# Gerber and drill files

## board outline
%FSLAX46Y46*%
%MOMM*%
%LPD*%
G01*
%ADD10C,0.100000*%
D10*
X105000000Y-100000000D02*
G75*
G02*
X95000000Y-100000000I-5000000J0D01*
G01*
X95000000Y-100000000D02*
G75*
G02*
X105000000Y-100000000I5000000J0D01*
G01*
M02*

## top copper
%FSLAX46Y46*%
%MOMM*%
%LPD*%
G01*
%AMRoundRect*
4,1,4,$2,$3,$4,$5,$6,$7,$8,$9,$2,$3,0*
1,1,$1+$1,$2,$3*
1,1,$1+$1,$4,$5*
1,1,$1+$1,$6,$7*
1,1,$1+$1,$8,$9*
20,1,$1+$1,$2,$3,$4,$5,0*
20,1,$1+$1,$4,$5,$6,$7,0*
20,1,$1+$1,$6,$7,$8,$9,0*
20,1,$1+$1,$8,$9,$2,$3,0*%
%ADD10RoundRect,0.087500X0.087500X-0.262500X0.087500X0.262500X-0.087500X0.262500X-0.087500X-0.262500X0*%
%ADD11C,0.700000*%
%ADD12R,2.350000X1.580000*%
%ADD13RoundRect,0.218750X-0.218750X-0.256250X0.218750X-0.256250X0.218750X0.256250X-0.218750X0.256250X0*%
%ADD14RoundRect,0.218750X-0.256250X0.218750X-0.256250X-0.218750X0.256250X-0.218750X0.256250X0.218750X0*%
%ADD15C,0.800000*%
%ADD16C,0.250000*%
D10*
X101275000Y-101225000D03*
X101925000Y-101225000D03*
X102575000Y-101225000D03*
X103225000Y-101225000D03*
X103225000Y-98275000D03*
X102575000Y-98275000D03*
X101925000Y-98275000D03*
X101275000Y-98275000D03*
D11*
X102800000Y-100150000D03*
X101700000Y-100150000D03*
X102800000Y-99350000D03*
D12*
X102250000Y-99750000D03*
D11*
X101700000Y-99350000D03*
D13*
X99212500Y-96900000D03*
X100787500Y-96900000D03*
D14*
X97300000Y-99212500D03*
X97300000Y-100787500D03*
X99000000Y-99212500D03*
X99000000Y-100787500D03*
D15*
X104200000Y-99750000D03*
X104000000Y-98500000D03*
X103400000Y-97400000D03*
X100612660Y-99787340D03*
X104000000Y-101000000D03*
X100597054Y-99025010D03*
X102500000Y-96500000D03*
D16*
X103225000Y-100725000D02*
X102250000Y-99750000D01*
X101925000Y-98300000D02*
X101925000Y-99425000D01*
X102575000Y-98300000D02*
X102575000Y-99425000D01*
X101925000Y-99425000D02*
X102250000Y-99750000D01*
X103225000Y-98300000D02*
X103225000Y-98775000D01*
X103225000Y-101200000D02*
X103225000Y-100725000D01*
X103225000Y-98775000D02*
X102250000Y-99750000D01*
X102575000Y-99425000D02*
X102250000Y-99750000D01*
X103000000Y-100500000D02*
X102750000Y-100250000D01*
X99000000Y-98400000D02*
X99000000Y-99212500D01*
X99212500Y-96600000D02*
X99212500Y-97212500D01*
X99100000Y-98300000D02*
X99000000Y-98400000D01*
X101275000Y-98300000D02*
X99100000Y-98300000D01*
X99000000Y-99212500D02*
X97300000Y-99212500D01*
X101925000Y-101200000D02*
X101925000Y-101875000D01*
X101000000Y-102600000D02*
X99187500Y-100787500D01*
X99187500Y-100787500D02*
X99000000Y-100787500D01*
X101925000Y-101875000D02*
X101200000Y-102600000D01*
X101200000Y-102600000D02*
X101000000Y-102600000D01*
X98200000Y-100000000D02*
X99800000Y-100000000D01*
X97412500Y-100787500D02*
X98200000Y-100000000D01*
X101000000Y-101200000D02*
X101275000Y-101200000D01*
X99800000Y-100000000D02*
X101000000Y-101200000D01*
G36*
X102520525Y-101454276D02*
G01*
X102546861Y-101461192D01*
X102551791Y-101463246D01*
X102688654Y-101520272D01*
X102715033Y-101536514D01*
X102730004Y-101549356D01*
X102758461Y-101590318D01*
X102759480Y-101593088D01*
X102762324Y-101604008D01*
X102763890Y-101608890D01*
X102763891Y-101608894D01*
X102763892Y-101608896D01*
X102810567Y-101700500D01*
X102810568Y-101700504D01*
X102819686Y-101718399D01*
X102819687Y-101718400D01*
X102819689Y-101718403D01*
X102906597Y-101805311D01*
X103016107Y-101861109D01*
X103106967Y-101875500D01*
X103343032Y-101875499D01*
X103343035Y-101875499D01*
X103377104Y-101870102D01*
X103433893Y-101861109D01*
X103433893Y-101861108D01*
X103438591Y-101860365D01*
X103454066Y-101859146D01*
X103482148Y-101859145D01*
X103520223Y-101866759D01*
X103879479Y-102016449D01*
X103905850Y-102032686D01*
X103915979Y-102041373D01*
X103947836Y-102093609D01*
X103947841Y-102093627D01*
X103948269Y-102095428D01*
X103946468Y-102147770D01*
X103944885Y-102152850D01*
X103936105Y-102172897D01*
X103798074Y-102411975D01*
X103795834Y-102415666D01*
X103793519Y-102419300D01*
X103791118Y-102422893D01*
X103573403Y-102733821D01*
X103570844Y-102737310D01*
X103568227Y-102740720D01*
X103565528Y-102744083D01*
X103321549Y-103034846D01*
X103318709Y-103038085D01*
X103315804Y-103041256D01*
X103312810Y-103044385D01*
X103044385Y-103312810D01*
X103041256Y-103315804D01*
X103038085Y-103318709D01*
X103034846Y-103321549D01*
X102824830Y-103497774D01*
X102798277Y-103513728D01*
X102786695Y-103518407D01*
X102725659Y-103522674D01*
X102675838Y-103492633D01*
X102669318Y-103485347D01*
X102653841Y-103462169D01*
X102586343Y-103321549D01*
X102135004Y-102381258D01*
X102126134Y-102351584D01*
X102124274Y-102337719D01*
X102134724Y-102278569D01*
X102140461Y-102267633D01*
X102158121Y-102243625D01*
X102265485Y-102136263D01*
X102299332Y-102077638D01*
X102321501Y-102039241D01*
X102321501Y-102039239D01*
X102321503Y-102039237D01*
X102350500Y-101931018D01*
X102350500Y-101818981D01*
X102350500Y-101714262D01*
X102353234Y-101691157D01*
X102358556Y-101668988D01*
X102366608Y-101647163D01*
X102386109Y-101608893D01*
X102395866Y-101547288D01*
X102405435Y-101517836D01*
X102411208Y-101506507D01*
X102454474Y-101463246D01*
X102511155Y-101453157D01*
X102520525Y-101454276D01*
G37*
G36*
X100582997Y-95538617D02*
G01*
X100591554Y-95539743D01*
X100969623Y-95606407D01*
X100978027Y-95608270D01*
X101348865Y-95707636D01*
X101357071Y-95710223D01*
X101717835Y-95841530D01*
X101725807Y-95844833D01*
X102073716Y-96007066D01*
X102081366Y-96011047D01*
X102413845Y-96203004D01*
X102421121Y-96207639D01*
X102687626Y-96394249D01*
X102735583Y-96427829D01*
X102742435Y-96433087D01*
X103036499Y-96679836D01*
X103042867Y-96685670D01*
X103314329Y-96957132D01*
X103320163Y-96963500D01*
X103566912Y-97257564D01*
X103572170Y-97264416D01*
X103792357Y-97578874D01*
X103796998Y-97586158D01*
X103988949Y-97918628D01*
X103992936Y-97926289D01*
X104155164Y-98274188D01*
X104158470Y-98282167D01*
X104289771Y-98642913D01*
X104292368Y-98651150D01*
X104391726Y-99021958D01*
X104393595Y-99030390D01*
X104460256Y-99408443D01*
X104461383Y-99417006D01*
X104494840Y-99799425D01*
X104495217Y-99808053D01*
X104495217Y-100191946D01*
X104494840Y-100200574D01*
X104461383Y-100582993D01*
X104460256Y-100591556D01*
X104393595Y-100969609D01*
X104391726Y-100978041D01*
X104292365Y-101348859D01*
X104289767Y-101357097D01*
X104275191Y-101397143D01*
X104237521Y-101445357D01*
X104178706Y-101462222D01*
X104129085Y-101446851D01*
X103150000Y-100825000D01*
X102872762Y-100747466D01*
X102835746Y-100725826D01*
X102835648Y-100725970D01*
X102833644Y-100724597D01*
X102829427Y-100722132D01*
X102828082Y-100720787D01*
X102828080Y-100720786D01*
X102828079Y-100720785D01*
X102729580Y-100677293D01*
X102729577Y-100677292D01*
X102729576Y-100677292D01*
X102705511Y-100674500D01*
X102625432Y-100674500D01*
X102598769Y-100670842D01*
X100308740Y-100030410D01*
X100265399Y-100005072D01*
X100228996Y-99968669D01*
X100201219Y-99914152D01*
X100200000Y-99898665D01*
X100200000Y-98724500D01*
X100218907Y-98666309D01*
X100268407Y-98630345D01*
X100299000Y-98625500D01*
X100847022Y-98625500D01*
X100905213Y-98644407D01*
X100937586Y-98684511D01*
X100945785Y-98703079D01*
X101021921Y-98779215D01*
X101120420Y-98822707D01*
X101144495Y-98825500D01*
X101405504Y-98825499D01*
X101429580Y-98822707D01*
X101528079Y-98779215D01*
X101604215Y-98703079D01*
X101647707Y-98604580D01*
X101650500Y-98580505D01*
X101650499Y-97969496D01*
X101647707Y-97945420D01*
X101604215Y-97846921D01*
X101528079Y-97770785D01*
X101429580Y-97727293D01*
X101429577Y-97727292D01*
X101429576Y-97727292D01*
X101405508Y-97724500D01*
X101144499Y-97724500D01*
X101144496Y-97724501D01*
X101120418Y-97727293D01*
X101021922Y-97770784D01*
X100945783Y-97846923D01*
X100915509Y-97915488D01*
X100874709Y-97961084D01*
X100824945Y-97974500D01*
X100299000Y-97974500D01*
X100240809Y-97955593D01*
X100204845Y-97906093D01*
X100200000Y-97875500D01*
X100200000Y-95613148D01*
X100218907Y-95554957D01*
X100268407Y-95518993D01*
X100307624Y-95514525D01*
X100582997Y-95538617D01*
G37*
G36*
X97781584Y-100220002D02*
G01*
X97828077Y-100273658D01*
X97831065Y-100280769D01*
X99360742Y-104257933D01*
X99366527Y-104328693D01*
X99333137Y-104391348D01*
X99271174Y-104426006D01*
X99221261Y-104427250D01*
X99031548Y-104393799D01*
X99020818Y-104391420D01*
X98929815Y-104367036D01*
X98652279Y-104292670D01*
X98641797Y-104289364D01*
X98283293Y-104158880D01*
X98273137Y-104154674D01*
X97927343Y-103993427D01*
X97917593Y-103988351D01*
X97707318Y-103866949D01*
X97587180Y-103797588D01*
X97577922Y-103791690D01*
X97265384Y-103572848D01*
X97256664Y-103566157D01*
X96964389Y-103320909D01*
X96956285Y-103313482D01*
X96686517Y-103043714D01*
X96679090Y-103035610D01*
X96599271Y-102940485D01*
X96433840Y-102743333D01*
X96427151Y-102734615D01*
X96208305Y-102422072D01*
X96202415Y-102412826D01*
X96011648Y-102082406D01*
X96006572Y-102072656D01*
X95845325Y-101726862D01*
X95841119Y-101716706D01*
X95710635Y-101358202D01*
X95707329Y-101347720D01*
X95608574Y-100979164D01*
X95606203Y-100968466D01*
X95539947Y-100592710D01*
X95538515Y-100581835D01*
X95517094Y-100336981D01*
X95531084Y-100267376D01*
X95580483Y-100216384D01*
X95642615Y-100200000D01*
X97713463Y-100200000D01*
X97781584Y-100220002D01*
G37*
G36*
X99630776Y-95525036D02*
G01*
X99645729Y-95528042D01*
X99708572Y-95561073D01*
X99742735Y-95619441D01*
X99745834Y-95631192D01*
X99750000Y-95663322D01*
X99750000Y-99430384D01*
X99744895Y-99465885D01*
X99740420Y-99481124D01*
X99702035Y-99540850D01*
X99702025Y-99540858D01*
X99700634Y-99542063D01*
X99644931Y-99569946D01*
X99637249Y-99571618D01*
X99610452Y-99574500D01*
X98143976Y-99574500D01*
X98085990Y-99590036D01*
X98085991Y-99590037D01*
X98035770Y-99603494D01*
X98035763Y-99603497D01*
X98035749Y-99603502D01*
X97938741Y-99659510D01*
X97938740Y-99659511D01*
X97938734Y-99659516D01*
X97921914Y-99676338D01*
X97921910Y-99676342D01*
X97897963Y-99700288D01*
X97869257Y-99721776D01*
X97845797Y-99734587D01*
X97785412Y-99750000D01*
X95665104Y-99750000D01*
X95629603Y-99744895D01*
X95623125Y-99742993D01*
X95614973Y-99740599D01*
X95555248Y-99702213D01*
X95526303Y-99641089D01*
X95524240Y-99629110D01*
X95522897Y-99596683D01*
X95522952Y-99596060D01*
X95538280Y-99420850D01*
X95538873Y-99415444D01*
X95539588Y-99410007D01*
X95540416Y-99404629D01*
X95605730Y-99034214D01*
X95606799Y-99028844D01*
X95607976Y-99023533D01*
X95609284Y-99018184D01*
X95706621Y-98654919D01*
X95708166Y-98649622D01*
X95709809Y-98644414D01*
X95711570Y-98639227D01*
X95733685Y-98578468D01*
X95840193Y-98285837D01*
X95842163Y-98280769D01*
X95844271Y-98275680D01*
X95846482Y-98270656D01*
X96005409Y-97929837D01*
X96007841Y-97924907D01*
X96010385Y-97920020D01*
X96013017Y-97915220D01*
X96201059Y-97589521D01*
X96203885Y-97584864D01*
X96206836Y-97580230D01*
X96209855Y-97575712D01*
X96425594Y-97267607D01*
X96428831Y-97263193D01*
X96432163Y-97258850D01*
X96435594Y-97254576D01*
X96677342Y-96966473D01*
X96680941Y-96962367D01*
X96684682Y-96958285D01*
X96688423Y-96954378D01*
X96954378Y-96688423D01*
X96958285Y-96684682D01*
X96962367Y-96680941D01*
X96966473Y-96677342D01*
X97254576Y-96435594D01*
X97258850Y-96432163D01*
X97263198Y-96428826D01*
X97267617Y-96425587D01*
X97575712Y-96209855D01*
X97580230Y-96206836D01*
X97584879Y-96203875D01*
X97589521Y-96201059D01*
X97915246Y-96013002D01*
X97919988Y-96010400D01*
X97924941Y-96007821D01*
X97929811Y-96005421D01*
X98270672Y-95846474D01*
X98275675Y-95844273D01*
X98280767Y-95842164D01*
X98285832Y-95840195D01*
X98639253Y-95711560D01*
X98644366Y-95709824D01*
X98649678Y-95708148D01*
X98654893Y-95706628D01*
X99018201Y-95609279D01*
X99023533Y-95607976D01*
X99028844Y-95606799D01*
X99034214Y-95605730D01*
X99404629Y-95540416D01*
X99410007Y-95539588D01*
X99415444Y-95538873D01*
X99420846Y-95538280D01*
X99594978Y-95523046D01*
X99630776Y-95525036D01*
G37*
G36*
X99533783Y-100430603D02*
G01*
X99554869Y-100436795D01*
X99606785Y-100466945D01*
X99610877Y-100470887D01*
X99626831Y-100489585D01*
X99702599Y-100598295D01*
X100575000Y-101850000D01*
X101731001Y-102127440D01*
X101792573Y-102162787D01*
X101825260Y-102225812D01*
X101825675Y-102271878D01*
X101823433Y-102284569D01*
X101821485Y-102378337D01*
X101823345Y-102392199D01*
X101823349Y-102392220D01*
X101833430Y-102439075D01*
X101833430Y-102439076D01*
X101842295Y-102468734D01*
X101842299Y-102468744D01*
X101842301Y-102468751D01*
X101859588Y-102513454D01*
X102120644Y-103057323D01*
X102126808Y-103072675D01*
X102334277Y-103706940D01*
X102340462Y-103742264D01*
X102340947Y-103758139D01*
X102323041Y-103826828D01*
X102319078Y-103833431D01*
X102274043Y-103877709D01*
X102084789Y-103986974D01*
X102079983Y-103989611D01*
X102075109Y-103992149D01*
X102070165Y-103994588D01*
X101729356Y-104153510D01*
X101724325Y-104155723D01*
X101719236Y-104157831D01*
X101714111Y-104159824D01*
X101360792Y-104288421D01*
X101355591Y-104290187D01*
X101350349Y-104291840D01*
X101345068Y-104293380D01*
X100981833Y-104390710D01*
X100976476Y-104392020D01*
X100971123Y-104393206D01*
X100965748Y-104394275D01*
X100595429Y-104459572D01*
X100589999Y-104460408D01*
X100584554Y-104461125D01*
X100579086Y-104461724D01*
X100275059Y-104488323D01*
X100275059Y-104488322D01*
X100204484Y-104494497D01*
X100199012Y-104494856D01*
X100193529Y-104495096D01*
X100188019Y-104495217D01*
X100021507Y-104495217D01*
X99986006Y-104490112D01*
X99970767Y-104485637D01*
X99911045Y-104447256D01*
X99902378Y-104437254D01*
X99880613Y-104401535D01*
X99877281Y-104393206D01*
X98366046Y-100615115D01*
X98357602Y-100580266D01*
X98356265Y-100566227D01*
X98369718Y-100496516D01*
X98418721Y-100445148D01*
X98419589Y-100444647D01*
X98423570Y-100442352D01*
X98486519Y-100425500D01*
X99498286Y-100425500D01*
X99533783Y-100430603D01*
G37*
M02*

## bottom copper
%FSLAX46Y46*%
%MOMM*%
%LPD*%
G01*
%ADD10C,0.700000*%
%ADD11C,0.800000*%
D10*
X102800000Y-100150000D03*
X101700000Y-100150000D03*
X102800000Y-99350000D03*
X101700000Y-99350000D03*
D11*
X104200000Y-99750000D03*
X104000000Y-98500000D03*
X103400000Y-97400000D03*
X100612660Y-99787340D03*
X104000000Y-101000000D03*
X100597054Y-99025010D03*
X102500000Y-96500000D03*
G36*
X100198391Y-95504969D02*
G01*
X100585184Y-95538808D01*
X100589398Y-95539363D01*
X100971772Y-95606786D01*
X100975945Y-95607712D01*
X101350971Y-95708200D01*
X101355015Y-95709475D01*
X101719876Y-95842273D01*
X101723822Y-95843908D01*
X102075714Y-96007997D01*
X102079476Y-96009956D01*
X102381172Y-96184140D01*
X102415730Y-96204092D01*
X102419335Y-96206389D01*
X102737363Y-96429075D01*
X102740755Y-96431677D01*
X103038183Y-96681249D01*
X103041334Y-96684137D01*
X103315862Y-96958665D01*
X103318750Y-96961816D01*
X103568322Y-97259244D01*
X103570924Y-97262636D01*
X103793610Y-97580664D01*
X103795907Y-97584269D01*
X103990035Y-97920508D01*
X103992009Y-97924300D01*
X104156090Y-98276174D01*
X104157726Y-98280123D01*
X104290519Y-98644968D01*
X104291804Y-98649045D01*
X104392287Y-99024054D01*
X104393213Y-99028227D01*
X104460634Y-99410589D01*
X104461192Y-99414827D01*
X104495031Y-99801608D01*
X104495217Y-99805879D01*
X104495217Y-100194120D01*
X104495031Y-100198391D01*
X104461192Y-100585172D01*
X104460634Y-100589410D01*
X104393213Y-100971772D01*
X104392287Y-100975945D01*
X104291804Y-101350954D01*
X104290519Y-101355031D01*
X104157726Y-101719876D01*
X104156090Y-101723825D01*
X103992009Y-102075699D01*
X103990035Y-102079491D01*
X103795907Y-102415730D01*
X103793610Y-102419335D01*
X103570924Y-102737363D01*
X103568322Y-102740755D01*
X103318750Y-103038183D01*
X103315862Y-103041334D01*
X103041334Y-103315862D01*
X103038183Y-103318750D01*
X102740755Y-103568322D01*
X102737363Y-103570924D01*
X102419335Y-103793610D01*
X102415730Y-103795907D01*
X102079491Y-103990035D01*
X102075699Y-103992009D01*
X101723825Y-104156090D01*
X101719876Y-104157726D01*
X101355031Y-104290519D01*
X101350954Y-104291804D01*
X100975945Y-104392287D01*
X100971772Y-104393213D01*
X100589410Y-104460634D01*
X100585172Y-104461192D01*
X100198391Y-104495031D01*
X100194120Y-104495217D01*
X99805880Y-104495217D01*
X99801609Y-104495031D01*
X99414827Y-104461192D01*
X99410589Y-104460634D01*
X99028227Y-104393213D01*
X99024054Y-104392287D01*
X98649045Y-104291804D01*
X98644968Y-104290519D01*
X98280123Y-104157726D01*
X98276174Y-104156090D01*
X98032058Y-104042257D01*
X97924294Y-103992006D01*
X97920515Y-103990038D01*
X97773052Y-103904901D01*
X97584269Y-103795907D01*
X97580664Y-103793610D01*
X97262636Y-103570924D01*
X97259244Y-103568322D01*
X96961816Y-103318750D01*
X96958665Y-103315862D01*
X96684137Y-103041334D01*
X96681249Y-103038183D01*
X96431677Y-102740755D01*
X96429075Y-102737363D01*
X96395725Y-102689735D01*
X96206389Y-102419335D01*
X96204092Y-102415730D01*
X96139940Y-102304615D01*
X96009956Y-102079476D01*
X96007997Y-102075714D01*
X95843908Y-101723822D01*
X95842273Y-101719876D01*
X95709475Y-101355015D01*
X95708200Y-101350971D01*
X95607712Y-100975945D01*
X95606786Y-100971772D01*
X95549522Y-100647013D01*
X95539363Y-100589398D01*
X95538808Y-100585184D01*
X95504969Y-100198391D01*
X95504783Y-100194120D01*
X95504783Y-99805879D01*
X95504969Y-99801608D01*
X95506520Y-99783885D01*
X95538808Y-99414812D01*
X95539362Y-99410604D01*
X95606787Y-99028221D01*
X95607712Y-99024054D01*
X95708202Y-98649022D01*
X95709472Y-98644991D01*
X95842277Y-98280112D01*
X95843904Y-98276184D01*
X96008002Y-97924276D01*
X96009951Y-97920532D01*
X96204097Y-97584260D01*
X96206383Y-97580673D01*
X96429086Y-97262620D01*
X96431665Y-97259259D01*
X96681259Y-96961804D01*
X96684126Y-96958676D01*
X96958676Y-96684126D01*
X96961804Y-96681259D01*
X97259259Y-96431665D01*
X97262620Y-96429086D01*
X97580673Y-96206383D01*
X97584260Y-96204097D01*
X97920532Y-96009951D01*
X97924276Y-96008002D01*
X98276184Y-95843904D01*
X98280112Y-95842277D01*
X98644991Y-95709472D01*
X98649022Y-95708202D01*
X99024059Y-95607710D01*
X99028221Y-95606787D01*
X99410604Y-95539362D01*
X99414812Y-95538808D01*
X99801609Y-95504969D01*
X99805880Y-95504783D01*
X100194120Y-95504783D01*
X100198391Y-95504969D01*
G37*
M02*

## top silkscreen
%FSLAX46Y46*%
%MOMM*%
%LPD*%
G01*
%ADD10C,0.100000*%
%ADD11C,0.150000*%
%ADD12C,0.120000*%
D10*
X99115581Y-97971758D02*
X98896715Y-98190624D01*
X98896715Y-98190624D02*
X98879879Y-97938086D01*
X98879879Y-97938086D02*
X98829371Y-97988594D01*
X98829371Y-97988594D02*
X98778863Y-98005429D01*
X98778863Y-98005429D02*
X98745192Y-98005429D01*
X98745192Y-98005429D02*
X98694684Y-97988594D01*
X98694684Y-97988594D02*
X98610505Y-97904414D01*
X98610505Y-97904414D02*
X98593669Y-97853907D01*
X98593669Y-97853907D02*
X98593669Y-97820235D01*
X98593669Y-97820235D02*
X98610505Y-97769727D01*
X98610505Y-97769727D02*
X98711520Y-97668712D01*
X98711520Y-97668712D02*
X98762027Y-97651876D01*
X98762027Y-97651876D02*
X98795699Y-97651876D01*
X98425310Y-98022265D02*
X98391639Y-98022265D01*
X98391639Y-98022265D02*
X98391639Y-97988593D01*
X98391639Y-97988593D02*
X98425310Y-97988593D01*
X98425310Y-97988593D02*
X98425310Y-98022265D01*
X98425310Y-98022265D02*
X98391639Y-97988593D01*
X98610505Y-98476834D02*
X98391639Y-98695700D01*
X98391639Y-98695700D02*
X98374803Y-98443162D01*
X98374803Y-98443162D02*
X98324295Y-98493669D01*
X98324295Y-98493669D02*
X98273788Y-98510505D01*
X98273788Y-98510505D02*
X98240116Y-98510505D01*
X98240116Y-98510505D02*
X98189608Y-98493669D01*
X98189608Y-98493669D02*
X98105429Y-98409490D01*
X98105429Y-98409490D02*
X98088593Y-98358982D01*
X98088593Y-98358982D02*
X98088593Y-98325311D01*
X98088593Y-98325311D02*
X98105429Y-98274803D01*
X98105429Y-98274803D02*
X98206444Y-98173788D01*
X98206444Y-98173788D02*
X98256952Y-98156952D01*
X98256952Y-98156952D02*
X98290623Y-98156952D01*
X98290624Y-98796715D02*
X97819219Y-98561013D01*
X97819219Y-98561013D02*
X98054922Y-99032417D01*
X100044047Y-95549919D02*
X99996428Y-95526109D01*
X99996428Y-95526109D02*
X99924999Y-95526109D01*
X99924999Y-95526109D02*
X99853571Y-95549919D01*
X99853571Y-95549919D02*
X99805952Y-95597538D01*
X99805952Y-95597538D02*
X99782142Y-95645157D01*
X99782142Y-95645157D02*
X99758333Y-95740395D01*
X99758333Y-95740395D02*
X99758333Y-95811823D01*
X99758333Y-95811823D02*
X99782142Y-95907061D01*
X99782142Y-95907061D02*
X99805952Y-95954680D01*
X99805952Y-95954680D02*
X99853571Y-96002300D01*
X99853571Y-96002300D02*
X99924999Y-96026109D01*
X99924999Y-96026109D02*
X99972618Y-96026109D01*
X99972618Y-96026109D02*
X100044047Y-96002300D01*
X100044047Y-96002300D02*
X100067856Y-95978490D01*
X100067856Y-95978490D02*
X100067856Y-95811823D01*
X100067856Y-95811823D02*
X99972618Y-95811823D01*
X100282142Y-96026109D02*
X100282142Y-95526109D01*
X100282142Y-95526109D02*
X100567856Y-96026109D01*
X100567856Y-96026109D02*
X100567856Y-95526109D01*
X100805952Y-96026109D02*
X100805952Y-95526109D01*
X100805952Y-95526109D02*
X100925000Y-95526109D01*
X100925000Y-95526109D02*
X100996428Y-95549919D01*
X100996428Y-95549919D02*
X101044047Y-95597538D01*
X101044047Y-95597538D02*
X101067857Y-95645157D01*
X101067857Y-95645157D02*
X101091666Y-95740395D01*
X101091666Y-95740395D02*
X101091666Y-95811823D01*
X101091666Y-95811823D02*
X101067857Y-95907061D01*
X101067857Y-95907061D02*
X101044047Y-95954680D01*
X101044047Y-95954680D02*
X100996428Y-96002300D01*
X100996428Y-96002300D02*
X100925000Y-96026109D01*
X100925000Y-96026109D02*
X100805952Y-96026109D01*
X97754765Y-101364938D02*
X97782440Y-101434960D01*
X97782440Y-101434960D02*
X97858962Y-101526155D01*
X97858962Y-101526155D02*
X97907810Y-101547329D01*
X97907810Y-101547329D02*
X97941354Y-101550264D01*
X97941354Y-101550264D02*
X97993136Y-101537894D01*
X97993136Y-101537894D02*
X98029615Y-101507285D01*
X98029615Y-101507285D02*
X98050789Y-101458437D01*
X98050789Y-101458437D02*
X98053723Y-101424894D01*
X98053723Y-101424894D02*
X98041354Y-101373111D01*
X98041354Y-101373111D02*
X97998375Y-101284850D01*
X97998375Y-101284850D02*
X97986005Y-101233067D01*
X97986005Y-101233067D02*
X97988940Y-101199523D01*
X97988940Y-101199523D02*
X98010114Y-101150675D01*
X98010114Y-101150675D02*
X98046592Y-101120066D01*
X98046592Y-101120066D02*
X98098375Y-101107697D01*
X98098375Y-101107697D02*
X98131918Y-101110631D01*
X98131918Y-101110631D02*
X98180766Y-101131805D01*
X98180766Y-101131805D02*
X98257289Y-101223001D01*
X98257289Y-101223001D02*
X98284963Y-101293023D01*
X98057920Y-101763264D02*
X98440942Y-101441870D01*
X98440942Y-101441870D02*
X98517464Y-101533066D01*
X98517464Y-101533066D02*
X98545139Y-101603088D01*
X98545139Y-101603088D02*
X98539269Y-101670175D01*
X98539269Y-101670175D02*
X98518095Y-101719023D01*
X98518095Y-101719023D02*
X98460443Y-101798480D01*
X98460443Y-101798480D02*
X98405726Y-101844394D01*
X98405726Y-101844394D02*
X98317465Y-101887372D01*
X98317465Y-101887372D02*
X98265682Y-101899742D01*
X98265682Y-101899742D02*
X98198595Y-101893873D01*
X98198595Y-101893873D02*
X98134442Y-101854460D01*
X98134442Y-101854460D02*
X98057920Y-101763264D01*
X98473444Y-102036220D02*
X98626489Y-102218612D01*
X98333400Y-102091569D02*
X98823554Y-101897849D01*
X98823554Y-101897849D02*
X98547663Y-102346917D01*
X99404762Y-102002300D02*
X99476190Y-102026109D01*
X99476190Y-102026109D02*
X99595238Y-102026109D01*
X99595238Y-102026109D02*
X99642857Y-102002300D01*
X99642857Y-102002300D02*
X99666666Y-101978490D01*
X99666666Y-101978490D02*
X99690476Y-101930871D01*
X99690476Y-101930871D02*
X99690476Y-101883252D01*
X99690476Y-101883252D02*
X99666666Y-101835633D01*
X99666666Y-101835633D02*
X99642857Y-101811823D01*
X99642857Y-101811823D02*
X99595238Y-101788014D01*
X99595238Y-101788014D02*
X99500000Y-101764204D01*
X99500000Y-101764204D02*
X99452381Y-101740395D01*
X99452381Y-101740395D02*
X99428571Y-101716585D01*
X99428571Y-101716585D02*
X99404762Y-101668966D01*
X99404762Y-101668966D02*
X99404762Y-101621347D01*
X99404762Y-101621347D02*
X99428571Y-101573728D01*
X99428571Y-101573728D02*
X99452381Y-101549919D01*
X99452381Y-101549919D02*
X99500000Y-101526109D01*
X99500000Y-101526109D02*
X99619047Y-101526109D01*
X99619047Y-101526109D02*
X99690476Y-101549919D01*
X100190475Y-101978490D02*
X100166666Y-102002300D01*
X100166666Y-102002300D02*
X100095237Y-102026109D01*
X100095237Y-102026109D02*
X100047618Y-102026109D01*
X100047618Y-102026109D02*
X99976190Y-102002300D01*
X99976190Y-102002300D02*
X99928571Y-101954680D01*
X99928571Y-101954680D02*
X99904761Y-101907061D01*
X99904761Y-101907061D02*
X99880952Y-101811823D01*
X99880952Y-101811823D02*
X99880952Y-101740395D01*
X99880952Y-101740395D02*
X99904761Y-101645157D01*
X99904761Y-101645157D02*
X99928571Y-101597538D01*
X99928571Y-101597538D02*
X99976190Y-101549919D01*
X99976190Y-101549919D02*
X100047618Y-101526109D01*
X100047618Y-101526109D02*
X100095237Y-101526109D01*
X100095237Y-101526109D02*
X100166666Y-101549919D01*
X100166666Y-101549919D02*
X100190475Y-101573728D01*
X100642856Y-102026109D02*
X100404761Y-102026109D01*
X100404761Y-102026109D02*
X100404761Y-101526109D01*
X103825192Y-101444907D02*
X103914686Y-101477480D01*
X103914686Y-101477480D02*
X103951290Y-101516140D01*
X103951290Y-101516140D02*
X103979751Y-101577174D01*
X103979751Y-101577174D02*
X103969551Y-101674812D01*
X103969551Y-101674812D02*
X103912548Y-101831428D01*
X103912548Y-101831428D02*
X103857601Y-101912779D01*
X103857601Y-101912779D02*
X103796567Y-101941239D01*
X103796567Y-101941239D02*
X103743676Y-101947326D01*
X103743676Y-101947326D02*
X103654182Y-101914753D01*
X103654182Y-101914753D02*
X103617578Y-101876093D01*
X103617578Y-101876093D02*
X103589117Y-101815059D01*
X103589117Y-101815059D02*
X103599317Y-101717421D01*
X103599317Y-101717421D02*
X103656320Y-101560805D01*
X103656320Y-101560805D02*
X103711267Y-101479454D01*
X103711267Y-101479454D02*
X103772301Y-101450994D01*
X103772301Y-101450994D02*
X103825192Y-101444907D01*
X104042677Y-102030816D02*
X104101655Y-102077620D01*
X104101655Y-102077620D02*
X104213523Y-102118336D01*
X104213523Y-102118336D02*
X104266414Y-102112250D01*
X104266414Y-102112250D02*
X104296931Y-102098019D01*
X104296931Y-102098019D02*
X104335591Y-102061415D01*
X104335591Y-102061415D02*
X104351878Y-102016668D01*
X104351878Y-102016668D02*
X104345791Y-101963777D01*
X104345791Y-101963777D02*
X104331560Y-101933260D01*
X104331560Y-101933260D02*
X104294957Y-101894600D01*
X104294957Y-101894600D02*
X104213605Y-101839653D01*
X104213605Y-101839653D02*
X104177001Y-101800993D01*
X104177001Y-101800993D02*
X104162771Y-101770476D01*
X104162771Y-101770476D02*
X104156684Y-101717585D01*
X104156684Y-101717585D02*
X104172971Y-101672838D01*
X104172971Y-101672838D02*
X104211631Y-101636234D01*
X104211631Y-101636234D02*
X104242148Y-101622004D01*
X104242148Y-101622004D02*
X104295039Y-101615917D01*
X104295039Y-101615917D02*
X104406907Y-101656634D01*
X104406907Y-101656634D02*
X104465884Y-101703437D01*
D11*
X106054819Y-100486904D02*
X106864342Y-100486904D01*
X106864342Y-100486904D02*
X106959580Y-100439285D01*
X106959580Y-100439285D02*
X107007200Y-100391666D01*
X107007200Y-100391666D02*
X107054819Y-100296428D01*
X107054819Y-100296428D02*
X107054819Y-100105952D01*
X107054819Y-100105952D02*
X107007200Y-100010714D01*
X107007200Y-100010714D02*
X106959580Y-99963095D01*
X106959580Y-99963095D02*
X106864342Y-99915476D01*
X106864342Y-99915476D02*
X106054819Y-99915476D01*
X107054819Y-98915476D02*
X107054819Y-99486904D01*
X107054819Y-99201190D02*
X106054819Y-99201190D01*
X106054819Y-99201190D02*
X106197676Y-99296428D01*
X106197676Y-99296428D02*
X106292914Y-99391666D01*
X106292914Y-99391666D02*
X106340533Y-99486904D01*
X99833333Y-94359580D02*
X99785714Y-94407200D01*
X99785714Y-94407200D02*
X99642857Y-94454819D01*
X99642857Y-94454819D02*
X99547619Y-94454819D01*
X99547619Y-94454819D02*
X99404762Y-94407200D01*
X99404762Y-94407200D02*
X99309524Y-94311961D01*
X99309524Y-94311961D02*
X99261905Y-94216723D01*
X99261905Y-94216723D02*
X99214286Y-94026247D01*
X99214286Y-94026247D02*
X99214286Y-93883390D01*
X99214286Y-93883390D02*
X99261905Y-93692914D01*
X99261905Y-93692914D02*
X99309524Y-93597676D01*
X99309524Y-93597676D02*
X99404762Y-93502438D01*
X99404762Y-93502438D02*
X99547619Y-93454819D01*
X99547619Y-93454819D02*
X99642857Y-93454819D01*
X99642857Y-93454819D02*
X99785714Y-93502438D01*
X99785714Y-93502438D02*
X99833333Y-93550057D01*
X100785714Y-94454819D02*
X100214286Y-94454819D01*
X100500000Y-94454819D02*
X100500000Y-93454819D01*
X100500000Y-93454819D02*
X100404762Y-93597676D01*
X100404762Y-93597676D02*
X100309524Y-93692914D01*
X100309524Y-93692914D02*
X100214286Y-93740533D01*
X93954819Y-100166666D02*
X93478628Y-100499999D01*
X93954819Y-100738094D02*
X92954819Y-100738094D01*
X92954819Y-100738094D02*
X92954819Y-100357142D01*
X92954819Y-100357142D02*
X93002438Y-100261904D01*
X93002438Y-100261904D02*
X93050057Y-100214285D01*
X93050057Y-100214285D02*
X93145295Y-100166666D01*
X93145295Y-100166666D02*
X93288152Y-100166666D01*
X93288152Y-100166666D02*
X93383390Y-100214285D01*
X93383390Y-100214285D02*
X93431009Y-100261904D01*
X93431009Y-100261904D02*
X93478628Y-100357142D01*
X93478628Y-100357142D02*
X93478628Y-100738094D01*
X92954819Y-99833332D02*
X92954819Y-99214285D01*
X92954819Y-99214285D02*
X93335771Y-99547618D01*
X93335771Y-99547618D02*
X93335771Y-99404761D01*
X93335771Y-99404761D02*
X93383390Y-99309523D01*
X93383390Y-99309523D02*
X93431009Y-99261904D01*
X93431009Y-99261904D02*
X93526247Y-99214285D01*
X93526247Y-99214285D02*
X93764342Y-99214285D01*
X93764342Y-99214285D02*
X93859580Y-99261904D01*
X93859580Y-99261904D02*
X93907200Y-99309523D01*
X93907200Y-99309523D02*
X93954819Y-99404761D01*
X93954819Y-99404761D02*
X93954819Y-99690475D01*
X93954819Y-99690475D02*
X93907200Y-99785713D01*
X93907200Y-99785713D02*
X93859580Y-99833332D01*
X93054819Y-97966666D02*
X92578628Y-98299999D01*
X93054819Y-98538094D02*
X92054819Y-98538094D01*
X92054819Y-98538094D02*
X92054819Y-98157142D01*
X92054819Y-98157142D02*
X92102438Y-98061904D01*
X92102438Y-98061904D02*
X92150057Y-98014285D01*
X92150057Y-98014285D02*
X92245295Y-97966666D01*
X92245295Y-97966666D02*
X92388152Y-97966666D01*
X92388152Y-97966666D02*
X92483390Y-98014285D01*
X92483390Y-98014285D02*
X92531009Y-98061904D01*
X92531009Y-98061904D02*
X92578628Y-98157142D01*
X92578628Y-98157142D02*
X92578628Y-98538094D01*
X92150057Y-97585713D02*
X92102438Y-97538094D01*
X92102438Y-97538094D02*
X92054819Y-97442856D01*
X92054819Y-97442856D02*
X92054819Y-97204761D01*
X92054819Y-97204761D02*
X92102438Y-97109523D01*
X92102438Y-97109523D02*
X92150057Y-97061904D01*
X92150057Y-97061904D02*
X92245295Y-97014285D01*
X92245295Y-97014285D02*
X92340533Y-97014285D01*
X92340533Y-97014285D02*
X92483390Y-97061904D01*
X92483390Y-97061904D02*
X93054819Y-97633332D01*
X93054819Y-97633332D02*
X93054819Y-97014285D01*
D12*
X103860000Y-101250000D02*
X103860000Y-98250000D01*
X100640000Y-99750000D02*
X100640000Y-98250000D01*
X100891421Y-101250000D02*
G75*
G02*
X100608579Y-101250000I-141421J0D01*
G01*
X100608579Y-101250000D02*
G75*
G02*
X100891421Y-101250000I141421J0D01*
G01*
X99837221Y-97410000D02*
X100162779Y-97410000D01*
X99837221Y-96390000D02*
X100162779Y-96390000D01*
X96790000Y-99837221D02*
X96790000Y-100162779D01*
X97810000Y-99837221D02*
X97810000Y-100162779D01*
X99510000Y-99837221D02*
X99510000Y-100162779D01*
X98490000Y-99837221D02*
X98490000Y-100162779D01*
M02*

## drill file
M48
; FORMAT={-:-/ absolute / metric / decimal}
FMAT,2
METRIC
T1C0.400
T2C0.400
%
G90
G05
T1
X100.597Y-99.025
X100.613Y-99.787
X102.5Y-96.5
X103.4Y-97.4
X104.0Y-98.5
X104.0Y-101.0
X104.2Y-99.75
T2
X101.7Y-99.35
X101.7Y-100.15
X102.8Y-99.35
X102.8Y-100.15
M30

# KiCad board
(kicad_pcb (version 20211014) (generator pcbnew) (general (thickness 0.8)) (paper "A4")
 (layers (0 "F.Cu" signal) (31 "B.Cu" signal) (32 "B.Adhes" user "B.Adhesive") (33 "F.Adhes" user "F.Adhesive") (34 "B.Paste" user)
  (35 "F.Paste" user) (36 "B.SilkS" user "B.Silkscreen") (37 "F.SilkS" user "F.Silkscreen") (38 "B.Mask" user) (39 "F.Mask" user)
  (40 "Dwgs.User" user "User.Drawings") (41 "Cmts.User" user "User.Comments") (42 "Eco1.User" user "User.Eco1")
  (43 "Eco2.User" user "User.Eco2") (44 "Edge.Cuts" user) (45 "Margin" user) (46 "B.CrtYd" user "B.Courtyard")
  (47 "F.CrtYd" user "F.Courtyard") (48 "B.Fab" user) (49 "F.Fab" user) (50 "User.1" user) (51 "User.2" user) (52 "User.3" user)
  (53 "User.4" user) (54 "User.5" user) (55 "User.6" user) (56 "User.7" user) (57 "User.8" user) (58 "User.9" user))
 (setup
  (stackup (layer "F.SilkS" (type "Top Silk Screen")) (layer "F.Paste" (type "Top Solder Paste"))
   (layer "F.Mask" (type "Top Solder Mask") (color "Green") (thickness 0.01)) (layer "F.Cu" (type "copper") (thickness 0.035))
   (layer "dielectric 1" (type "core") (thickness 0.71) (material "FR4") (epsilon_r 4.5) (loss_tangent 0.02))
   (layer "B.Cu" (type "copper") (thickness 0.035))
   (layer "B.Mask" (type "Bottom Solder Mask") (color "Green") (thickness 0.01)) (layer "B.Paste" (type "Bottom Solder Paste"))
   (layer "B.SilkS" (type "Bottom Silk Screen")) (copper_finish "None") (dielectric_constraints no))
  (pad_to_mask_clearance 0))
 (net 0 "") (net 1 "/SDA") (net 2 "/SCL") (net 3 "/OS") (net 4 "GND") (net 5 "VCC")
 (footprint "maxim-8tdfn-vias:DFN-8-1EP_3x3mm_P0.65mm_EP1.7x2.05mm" (layer "F.Cu") (at 102.25 99.75 90)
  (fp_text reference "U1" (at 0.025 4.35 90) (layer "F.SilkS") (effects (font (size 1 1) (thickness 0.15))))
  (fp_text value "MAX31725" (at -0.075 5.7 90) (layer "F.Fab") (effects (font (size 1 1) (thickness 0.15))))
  (fp_line (start -1.5 1.61) (end 1.5 1.61) (layer "F.SilkS") (width 0.12))
  (fp_line (start 0 -1.61) (end 1.5 -1.61) (layer "F.SilkS") (width 0.12))
  (fp_circle (center -1.5 -1.5) (end -1.4 -1.4) (layer "F.SilkS") (width 0.12) (fill none))
  (pad "" smd roundrect locked (at -0.425 -0.51 90) (size 0.69 0.83) (layers "F.Paste") (roundrect_rratio 0.25))
  (pad "" smd roundrect locked (at 0.425 -0.51 90) (size 0.69 0.83) (layers "F.Paste") (roundrect_rratio 0.25))
  (pad "" smd roundrect locked (at 0.425 0.51 90) (size 0.69 0.83) (layers "F.Paste") (roundrect_rratio 0.25))
  (pad "" smd roundrect locked (at -0.425 0.51 90) (size 0.69 0.83) (layers "F.Paste") (roundrect_rratio 0.25))
  (pad "1" smd roundrect locked (at -1.475 -0.975 90) (size 0.7 0.35) (layers "F.Cu" "F.Paste" "F.Mask") (roundrect_rratio 0.25)
   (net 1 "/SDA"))
  (pad "2" smd roundrect locked (at -1.475 -0.325 90) (size 0.7 0.35) (layers "F.Cu" "F.Paste" "F.Mask") (roundrect_rratio 0.25)
   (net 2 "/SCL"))
  (pad "3" smd roundrect locked (at -1.475 0.325 90) (size 0.7 0.35) (layers "F.Cu" "F.Paste" "F.Mask") (roundrect_rratio 0.25)
   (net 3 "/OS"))
  (pad "4" smd roundrect locked (at -1.475 0.975 90) (size 0.7 0.35) (layers "F.Cu" "F.Paste" "F.Mask") (roundrect_rratio 0.25)
   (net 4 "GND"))
  (pad "5" smd roundrect locked (at 1.475 0.975 90) (size 0.7 0.35) (layers "F.Cu" "F.Paste" "F.Mask") (roundrect_rratio 0.25) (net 4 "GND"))
  (pad "6" smd roundrect locked (at 1.475 0.325 90) (size 0.7 0.35) (layers "F.Cu" "F.Paste" "F.Mask") (roundrect_rratio 0.25) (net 4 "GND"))
  (pad "7" smd roundrect locked (at 1.475 -0.325 90) (size 0.7 0.35) (layers "F.Cu" "F.Paste" "F.Mask") (roundrect_rratio 0.25)
   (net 4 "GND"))
  (pad "8" smd roundrect locked (at 1.475 -0.975 90) (size 0.7 0.35) (layers "F.Cu" "F.Paste" "F.Mask") (roundrect_rratio 0.25)
   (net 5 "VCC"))
  (pad "9" thru_hole circle locked (at -0.4 0.55 90) (size 0.7 0.7) (drill 0.4) (layers *.Cu *.Mask) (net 4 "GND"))
  (pad "9" thru_hole circle locked (at -0.4 -0.55 90) (size 0.7 0.7) (drill 0.4) (layers *.Cu *.Mask) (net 4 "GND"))
  (pad "9" thru_hole circle locked (at 0.4 0.55 90) (size 0.7 0.7) (drill 0.4) (layers *.Cu *.Mask) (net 4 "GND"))
  (pad "9" smd rect locked (at 0 0 90) (size 1.58 2.35) (layers "F.Cu" "F.Mask") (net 4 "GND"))
  (pad "9" thru_hole circle locked (at 0.4 -0.55 90) (size 0.7 0.7) (drill 0.4) (layers *.Cu *.Mask) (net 4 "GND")))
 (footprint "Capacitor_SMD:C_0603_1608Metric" (layer "F.Cu") (at 100 96.9)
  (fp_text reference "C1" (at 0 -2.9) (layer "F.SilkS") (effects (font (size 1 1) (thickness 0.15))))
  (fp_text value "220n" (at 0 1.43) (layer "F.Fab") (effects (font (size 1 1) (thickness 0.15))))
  (fp_line (start -0.162779 0.51) (end 0.162779 0.51) (layer "F.SilkS") (width 0.12))
  (fp_line (start -0.162779 -0.51) (end 0.162779 -0.51) (layer "F.SilkS") (width 0.12))
  (pad "1" smd roundrect locked (at -0.7875 0) (size 0.875 0.95) (layers "F.Cu" "F.Paste" "F.Mask") (roundrect_rratio 0.25) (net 5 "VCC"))
  (pad "2" smd roundrect locked (at 0.7875 0) (size 0.875 0.95) (layers "F.Cu" "F.Paste" "F.Mask") (roundrect_rratio 0.25) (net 4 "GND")))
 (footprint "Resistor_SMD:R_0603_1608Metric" (layer "F.Cu") (at 97.3 100 -90)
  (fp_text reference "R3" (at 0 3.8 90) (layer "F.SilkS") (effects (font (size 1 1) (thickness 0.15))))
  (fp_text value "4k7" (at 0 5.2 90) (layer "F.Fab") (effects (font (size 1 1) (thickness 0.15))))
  (fp_line (start -0.162779 0.51) (end 0.162779 0.51) (layer "F.SilkS") (width 0.12))
  (fp_line (start -0.162779 -0.51) (end 0.162779 -0.51) (layer "F.SilkS") (width 0.12))
  (pad "1" smd roundrect locked (at -0.7875 0 270) (size 0.875 0.95) (layers "F.Cu" "F.Paste" "F.Mask") (roundrect_rratio 0.25)
   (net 5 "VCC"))
  (pad "2" smd roundrect locked (at 0.7875 0 270) (size 0.875 0.95) (layers "F.Cu" "F.Paste" "F.Mask") (roundrect_rratio 0.25)
   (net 1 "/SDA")))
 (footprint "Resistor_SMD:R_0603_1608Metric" (layer "F.Cu") (at 99 100 -90)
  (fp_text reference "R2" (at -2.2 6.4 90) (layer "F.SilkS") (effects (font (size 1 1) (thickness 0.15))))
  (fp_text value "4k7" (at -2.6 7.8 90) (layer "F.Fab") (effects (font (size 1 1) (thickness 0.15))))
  (fp_line (start -0.162779 -0.51) (end 0.162779 -0.51) (layer "F.SilkS") (width 0.12))
  (fp_line (start -0.162779 0.51) (end 0.162779 0.51) (layer "F.SilkS") (width 0.12))
  (pad "1" smd roundrect locked (at -0.7875 0 270) (size 0.875 0.95) (layers "F.Cu" "F.Paste" "F.Mask") (roundrect_rratio 0.25)
   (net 5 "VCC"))
  (pad "2" smd roundrect locked (at 0.7875 0 270) (size 0.875 0.95) (layers "F.Cu" "F.Paste" "F.Mask") (roundrect_rratio 0.25)
   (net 2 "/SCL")))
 (gr_circle (center 100 100) (end 105 100) (layer "Edge.Cuts") (width 0.1) (fill none))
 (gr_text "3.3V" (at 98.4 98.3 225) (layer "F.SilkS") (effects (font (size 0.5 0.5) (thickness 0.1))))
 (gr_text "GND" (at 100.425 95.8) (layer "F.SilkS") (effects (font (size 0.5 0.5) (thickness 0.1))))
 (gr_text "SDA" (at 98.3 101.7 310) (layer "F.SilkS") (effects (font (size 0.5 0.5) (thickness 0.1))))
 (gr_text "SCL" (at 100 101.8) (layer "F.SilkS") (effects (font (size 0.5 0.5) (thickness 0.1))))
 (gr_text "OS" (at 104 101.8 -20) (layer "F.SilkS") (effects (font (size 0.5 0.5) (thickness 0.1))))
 (segment (start 103.225 100.725) (end 102.25 99.75) (width 0.25) (layer "F.Cu") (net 4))
 (segment (start 101.925 98.3) (end 101.925 99.425) (width 0.25) (layer "F.Cu") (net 4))
 (segment (start 102.575 98.3) (end 102.575 99.425) (width 0.25) (layer "F.Cu") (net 4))
 (segment (start 101.925 99.425) (end 102.25 99.75) (width 0.25) (layer "F.Cu") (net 4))
 (segment (start 103.225 98.3) (end 103.225 98.775) (width 0.25) (layer "F.Cu") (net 4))
 (segment (start 103.225 101.2) (end 103.225 100.725) (width 0.25) (layer "F.Cu") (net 4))
 (segment (start 103.225 98.775) (end 102.25 99.75) (width 0.25) (layer "F.Cu") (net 4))
 (segment (start 102.575 99.425) (end 102.25 99.75) (width 0.25) (layer "F.Cu") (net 4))
 (segment (start 103 100.5) (end 102.75 100.25) (width 0.25) (layer "F.Cu") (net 4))
 (via (at 104.2 99.75) (size 0.8) (drill 0.4) (layers "F.Cu" "B.Cu") (free) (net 4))
 (via (at 104 98.5) (size 0.8) (drill 0.4) (layers "F.Cu" "B.Cu") (free) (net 4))
 (via (at 103.4 97.4) (size 0.8) (drill 0.4) (layers "F.Cu" "B.Cu") (free) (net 4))
 (via (at 100.61266 99.78734) (size 0.8) (drill 0.4) (layers "F.Cu" "B.Cu") (free) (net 4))
 (via (at 104 101) (size 0.8) (drill 0.4) (layers "F.Cu" "B.Cu") (free) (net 4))
 (via (at 100.597054 99.02501) (size 0.8) (drill 0.4) (layers "F.Cu" "B.Cu") (free) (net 4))
 (via (at 102.5 96.5) (size 0.8) (drill 0.4) (layers "F.Cu" "B.Cu") (free) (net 4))
 (segment (start 99 98.4) (end 99 99.2125) (width 0.25) (layer "F.Cu") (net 5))
 (segment (start 99.2125 96.6) (end 99.2125 97.2125) (width 0.25) (layer "F.Cu") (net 5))
 (segment (start 99.1 98.3) (end 99 98.4) (width 0.25) (layer "F.Cu") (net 5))
 (segment (start 101.275 98.3) (end 99.1 98.3) (width 0.25) (layer "F.Cu") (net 5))
 (segment (start 99 99.2125) (end 97.3 99.2125) (width 0.25) (layer "F.Cu") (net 5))
 (segment (start 101.925 101.2) (end 101.925 101.875) (width 0.25) (layer "F.Cu") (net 2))
 (segment (start 101 102.6) (end 99.1875 100.7875) (width 0.25) (layer "F.Cu") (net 2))
 (segment (start 99.1875 100.7875) (end 99 100.7875) (width 0.25) (layer "F.Cu") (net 2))
 (segment (start 101.925 101.875) (end 101.2 102.6) (width 0.25) (layer "F.Cu") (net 2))
 (segment (start 101.2 102.6) (end 101 102.6) (width 0.25) (layer "F.Cu") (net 2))
 (segment (start 98.2 100) (end 99.8 100) (width 0.25) (layer "F.Cu") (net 1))
 (segment (start 97.4125 100.7875) (end 98.2 100) (width 0.25) (layer "F.Cu") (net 1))
 (segment (start 101 101.2) (end 101.275 101.2) (width 0.25) (layer "F.Cu") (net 1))
 (segment (start 99.8 100) (end 101 101.2) (width 0.25) (layer "F.Cu") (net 1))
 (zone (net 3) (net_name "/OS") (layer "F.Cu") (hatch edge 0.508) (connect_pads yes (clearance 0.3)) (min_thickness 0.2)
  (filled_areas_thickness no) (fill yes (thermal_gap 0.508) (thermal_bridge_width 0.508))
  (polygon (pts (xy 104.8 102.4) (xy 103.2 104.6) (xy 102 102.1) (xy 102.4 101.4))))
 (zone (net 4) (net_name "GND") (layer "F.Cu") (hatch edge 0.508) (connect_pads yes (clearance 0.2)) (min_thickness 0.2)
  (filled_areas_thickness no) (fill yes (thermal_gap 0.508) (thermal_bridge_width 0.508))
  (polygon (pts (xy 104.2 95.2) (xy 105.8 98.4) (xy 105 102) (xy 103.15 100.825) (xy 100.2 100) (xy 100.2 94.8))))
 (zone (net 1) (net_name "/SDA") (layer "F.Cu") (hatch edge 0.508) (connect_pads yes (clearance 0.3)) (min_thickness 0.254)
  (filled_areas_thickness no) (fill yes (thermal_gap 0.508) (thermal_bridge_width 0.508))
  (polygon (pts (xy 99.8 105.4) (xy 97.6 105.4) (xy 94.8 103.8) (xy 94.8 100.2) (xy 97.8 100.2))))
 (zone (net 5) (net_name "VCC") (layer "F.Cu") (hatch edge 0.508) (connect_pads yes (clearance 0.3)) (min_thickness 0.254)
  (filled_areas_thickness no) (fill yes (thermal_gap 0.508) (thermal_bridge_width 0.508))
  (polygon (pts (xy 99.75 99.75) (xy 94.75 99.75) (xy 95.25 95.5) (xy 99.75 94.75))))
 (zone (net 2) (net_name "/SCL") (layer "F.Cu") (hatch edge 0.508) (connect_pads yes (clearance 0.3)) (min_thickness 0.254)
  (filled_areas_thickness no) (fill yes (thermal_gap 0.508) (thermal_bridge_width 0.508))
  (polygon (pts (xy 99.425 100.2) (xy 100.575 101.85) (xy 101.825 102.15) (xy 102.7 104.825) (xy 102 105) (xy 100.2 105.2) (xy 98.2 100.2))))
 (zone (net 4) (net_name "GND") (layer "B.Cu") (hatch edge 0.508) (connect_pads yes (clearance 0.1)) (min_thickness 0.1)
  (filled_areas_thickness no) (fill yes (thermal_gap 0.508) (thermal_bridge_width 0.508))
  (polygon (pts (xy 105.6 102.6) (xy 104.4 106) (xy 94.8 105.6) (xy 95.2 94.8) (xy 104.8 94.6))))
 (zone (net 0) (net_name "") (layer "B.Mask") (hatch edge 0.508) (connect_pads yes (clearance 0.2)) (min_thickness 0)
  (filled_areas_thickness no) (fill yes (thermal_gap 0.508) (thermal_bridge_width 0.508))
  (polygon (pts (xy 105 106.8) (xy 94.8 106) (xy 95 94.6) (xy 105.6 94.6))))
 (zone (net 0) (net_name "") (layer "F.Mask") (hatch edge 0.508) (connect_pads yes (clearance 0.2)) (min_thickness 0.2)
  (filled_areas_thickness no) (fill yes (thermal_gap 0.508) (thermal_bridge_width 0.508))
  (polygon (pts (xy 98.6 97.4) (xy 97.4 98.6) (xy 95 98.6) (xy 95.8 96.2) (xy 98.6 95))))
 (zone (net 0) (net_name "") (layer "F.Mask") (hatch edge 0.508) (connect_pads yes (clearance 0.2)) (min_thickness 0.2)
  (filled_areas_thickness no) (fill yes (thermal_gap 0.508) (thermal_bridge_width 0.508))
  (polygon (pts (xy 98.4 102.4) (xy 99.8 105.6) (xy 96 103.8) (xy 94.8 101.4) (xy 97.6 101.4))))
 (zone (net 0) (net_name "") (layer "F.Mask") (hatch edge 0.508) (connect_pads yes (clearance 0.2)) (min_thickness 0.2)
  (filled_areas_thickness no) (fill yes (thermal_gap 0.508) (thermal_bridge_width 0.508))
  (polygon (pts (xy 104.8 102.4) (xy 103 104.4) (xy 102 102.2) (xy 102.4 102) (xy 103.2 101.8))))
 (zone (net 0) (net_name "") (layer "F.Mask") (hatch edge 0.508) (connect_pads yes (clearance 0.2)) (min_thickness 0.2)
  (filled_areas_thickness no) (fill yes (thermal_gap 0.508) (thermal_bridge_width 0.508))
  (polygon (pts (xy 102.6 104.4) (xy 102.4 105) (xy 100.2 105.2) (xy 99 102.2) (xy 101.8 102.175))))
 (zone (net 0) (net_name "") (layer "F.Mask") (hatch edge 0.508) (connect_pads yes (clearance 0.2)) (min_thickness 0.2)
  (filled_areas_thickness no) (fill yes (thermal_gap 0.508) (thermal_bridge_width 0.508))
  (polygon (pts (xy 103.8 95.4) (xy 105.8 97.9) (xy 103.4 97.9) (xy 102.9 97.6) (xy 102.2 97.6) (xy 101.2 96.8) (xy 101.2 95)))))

